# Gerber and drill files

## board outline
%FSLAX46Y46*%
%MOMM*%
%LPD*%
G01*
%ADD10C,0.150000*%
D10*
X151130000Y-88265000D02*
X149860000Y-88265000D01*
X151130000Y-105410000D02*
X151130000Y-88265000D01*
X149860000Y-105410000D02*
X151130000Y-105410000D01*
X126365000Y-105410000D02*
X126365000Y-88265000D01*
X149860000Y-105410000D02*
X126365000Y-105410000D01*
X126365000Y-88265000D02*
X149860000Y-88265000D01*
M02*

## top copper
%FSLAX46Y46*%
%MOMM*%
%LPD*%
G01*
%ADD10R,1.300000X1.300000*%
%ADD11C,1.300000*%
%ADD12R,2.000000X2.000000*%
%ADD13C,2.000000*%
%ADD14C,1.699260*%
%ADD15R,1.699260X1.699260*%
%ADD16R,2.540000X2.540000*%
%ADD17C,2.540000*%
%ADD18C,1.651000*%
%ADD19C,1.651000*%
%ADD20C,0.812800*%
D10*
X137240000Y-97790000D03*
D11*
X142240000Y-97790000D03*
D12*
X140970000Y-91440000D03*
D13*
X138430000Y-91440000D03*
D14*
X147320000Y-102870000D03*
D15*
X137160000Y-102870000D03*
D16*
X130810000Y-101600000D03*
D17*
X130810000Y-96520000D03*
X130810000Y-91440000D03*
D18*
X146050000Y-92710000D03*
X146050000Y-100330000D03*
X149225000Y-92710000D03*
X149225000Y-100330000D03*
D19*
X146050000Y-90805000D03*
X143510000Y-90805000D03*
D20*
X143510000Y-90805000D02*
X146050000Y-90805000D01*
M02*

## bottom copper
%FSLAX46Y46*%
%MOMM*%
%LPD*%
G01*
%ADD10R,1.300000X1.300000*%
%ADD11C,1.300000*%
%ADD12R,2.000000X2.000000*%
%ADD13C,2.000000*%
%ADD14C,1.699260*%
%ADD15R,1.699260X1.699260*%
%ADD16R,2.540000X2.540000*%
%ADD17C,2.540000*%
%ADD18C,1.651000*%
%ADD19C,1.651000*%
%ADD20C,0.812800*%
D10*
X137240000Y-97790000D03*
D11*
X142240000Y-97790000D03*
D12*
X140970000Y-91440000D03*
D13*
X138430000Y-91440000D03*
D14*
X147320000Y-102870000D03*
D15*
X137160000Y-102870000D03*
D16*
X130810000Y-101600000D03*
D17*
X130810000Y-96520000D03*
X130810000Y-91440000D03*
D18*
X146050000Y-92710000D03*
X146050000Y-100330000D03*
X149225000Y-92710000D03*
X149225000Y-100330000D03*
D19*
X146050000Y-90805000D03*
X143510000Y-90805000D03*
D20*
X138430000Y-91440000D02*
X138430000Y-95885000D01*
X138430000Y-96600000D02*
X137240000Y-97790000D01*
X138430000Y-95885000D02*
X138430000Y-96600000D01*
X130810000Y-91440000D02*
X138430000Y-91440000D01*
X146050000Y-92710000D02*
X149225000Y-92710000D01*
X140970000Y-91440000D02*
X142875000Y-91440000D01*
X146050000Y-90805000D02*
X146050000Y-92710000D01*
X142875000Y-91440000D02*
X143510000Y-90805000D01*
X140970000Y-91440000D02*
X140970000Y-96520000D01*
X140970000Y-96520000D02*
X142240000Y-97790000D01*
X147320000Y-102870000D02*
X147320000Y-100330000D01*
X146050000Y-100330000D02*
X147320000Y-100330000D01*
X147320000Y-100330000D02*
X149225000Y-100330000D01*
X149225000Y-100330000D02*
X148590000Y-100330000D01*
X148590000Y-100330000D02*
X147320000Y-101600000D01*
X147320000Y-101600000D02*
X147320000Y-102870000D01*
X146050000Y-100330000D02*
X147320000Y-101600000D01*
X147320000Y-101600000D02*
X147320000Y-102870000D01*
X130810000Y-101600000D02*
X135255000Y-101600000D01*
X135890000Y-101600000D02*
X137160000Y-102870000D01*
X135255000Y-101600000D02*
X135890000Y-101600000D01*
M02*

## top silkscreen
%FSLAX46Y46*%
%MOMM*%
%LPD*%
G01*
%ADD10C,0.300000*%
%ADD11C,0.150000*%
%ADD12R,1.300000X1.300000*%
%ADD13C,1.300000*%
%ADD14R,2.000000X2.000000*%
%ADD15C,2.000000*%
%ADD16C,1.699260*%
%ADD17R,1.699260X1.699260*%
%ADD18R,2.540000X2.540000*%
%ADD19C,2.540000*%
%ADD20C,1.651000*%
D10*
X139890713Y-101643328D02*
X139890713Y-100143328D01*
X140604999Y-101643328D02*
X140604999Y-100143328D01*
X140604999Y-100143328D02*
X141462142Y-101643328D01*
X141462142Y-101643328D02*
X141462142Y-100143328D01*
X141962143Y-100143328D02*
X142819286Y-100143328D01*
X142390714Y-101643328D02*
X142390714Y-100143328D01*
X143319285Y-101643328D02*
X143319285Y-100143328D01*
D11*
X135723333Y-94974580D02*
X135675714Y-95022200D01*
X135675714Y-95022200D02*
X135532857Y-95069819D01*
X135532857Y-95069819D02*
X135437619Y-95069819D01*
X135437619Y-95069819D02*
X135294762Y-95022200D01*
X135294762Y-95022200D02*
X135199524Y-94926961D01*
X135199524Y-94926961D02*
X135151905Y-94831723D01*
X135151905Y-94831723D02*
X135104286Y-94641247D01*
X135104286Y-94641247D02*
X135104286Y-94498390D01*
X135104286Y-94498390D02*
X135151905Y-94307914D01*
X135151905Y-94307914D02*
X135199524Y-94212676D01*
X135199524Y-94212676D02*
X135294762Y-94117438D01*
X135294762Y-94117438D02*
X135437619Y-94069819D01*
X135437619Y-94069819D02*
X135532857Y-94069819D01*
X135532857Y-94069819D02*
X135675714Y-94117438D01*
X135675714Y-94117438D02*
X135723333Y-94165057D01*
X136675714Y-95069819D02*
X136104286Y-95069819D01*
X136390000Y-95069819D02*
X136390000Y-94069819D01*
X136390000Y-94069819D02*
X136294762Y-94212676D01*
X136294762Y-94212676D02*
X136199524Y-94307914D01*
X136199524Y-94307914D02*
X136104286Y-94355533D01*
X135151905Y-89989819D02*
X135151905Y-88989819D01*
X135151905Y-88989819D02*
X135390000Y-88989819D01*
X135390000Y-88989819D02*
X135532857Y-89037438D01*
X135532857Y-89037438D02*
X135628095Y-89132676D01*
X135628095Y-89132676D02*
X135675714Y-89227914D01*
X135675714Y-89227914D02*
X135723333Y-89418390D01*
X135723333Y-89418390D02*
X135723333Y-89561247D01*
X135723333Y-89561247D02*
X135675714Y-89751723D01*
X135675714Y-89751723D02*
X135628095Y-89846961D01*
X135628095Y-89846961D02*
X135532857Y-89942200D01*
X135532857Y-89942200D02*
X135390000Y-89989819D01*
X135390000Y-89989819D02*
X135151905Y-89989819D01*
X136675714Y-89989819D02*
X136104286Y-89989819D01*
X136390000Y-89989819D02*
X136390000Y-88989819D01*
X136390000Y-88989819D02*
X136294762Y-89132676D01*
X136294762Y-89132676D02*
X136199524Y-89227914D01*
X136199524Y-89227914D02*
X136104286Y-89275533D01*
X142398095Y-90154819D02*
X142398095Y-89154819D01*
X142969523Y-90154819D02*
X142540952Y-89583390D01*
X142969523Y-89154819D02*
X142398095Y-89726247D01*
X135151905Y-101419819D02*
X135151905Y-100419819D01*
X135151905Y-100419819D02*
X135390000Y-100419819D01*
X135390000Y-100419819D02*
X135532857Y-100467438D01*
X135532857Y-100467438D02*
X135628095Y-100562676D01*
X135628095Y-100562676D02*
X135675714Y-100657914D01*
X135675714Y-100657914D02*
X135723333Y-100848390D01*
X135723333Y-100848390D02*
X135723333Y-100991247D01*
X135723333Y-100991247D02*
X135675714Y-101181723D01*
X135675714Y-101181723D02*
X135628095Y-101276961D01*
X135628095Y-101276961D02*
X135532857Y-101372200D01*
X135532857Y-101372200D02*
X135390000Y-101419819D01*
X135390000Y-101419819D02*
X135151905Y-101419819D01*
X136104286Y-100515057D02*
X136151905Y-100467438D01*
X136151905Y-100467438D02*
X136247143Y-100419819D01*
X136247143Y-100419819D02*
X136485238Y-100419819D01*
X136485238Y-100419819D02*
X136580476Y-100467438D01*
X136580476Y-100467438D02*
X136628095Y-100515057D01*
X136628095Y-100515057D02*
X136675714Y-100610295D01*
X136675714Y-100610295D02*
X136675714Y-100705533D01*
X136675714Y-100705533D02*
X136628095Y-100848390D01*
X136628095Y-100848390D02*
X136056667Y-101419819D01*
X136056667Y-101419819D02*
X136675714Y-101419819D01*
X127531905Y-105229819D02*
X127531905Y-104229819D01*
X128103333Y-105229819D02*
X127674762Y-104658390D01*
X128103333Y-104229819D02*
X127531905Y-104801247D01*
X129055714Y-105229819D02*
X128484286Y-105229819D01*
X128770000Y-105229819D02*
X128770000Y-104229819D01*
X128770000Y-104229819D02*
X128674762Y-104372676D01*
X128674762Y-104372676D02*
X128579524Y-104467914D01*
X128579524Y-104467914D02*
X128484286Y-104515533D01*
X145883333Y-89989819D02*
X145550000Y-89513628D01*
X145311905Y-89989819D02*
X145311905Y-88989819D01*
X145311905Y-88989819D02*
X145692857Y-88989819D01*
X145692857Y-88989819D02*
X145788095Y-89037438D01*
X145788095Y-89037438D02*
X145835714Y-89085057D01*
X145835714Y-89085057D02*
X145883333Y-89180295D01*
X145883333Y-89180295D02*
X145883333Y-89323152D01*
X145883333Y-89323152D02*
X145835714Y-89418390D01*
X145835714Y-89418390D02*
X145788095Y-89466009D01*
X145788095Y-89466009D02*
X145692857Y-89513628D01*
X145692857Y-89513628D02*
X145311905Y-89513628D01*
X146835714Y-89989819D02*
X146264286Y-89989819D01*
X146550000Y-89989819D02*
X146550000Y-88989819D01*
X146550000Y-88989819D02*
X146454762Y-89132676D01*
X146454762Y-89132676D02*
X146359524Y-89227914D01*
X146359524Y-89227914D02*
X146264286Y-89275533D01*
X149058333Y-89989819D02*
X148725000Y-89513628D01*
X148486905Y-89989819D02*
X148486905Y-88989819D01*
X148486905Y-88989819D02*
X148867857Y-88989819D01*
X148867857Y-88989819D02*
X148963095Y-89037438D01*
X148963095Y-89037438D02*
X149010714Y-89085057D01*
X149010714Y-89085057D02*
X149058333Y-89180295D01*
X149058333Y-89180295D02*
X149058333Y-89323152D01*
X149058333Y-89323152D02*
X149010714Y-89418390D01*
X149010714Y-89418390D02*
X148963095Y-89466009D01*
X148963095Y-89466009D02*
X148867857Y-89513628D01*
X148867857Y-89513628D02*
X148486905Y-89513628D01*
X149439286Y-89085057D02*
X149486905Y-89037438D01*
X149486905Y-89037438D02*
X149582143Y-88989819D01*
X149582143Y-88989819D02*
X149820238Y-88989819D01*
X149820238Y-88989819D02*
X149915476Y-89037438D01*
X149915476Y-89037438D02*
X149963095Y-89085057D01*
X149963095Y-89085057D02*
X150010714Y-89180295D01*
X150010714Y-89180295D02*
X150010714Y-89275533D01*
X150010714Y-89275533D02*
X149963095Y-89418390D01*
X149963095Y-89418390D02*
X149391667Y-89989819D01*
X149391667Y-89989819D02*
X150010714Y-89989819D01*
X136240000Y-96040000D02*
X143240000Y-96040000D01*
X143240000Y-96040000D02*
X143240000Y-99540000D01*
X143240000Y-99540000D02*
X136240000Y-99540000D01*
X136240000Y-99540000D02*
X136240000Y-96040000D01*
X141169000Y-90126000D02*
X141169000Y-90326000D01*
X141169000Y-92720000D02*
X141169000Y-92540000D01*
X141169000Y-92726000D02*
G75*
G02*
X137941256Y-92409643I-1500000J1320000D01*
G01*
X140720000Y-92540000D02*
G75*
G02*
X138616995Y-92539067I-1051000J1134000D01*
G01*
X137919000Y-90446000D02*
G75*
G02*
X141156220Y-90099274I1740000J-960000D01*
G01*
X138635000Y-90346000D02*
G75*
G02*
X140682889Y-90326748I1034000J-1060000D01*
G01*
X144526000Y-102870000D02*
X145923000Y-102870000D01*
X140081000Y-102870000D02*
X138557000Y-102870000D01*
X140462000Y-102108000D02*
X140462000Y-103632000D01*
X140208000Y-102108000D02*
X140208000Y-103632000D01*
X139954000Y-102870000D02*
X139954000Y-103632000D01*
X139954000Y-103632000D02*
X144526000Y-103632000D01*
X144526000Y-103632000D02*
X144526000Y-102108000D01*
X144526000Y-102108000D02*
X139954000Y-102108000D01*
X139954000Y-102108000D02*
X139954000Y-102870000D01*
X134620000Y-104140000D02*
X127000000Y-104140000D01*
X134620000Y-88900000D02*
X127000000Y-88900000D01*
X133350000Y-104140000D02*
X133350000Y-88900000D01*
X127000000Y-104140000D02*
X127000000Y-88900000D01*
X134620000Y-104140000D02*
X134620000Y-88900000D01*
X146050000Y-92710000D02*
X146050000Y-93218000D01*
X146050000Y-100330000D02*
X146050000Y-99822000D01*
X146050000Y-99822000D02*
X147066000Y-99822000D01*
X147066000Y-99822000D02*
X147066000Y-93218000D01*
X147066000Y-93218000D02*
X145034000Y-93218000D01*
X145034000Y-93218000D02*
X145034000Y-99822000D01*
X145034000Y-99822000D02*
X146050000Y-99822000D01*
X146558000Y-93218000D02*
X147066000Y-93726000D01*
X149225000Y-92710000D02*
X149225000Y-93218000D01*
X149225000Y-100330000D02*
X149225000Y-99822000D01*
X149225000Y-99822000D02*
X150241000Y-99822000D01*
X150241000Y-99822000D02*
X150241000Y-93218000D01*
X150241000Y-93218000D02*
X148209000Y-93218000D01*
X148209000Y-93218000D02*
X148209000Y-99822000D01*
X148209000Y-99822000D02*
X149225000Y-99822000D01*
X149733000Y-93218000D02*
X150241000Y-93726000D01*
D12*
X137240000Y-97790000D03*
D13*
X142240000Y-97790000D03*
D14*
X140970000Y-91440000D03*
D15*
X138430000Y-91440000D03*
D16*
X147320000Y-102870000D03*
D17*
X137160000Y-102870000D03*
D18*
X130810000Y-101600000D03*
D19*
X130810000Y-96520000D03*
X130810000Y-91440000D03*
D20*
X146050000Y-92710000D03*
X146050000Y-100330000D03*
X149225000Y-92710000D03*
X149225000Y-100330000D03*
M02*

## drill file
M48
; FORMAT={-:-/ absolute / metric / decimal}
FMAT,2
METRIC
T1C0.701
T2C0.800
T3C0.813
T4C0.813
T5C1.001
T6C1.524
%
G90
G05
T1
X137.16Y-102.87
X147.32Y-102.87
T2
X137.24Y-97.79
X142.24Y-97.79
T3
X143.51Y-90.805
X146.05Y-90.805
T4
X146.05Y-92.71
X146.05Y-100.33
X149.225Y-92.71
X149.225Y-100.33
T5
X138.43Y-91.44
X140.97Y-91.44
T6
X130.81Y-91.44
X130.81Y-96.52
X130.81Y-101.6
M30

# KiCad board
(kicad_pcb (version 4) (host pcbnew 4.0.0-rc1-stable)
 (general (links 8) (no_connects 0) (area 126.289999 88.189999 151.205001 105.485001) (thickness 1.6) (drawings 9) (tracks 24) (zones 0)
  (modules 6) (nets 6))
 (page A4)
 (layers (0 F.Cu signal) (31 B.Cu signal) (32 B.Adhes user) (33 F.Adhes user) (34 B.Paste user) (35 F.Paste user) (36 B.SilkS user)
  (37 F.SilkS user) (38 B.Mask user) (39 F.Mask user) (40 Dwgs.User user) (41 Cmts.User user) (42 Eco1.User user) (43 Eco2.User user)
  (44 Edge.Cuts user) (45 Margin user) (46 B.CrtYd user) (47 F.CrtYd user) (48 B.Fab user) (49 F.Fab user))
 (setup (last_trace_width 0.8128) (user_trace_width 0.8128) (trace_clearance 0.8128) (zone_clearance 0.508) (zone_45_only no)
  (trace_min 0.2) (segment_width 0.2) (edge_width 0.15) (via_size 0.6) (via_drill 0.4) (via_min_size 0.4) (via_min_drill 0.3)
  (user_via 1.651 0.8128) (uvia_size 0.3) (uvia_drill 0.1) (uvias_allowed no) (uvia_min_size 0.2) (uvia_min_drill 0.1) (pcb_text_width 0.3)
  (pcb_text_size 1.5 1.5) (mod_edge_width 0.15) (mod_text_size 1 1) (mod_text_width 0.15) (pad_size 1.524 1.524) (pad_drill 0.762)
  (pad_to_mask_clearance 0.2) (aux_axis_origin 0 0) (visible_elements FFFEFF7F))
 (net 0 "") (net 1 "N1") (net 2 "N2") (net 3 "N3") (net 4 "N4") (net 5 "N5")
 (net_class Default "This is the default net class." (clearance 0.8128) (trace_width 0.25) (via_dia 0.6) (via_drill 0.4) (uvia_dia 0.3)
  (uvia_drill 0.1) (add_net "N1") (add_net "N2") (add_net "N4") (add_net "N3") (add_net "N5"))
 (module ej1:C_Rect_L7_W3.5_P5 (layer F.Cu) (at 137.24 97.79)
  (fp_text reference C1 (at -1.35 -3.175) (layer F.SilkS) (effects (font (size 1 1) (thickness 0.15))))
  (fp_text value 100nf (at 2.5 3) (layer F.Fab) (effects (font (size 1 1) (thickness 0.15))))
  (fp_line (start -1 -1.75) (end 6 -1.75) (layer F.SilkS) (width 0.15))
  (fp_line (start 6 -1.75) (end 6 1.75) (layer F.SilkS) (width 0.15))
  (fp_line (start 6 1.75) (end -1 1.75) (layer F.SilkS) (width 0.15))
  (fp_line (start -1 1.75) (end -1 -1.75) (layer F.SilkS) (width 0.15))
  (pad 1 thru_hole rect (at 0 0) (size 1.3 1.3) (drill 0.8) (layers *.Cu *.Mask F.SilkS) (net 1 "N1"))
  (pad 2 thru_hole circle (at 5 0) (size 1.3 1.3) (drill 0.8) (layers *.Cu *.Mask F.SilkS) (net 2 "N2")))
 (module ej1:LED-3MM (layer F.Cu) (at 140.97 91.44 180)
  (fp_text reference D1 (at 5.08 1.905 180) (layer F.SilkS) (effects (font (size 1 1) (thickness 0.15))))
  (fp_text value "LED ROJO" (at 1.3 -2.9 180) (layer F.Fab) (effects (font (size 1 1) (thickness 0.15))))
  (fp_line (start -0.199 1.314) (end -0.199 1.114) (layer F.SilkS) (width 0.15))
  (fp_line (start -0.199 -1.28) (end -0.199 -1.1) (layer F.SilkS) (width 0.15))
  (fp_arc (start 1.301 0.034) (end -0.199 -1.286) (angle 108.5) (layer F.SilkS) (width 0.15))
  (fp_arc (start 1.301 0.034) (end 0.25 -1.1) (angle 85.7) (layer F.SilkS) (width 0.15))
  (fp_arc (start 1.311 0.034) (end 3.051 0.994) (angle 110) (layer F.SilkS) (width 0.15))
  (fp_arc (start 1.301 0.034) (end 2.335 1.094) (angle 87.5) (layer F.SilkS) (width 0.15))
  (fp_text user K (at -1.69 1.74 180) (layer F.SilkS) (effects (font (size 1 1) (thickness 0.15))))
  (pad 1 thru_hole rect (at 0 0 270) (size 2 2) (drill 1.00076) (layers *.Cu *.Mask F.SilkS) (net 2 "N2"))
  (pad 2 thru_hole circle (at 2.54 0 180) (size 2 2) (drill 1.00076) (layers *.Cu *.Mask F.SilkS) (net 1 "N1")))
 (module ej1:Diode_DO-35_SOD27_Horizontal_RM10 (layer F.Cu) (at 137.15948 102.87254)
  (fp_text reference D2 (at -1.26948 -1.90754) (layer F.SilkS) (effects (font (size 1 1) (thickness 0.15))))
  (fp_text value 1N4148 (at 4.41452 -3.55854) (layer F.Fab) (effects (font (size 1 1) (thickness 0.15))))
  (fp_line (start 7.36652 -0.00254) (end 8.76352 -0.00254) (layer F.SilkS) (width 0.15))
  (fp_line (start 2.92152 -0.00254) (end 1.39752 -0.00254) (layer F.SilkS) (width 0.15))
  (fp_line (start 3.30252 -0.76454) (end 3.30252 0.75946) (layer F.SilkS) (width 0.15))
  (fp_line (start 3.04852 -0.76454) (end 3.04852 0.75946) (layer F.SilkS) (width 0.15))
  (fp_line (start 2.79452 -0.00254) (end 2.79452 0.75946) (layer F.SilkS) (width 0.15))
  (fp_line (start 2.79452 0.75946) (end 7.36652 0.75946) (layer F.SilkS) (width 0.15))
  (fp_line (start 7.36652 0.75946) (end 7.36652 -0.76454) (layer F.SilkS) (width 0.15))
  (fp_line (start 7.36652 -0.76454) (end 2.79452 -0.76454) (layer F.SilkS) (width 0.15))
  (fp_line (start 2.79452 -0.76454) (end 2.79452 -0.00254) (layer F.SilkS) (width 0.15))
  (pad 2 thru_hole circle (at 10.16052 -0.00254 180) (size 1.69926 1.69926) (drill 0.70104) (layers *.Cu *.Mask F.SilkS) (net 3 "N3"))
  (pad 1 thru_hole rect (at 0.00052 -0.00254 180) (size 1.69926 1.69926) (drill 0.70104) (layers *.Cu *.Mask F.SilkS) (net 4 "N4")))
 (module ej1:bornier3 (layer F.Cu) (at 130.81 96.52 90)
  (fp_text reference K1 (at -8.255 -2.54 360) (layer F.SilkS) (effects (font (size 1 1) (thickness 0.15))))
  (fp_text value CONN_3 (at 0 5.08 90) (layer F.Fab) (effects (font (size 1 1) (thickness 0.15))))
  (fp_line (start -7.62 3.81) (end -7.62 -3.81) (layer F.SilkS) (width 0.15))
  (fp_line (start 7.62 3.81) (end 7.62 -3.81) (layer F.SilkS) (width 0.15))
  (fp_line (start -7.62 2.54) (end 7.62 2.54) (layer F.SilkS) (width 0.15))
  (fp_line (start -7.62 -3.81) (end 7.62 -3.81) (layer F.SilkS) (width 0.15))
  (fp_line (start -7.62 3.81) (end 7.62 3.81) (layer F.SilkS) (width 0.15))
  (pad 1 thru_hole rect (at -5.08 0 90) (size 2.54 2.54) (drill 1.524) (layers *.Cu *.Mask F.SilkS) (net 4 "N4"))
  (pad 2 thru_hole circle (at 0 0 90) (size 2.54 2.54) (drill 1.524) (layers *.Cu *.Mask F.SilkS) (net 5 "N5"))
  (pad 3 thru_hole circle (at 5.08 0 90) (size 2.54 2.54) (drill 1.524) (layers *.Cu *.Mask F.SilkS) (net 1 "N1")))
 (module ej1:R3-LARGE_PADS (layer F.Cu) (at 146.05 96.52 270)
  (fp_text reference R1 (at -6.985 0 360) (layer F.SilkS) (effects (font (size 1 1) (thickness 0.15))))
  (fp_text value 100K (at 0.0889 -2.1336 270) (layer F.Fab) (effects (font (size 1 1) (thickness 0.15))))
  (fp_line (start -3.81 0) (end -3.302 0) (layer F.SilkS) (width 0.15))
  (fp_line (start 3.81 0) (end 3.302 0) (layer F.SilkS) (width 0.15))
  (fp_line (start 3.302 0) (end 3.302 -1.016) (layer F.SilkS) (width 0.15))
  (fp_line (start 3.302 -1.016) (end -3.302 -1.016) (layer F.SilkS) (width 0.15))
  (fp_line (start -3.302 -1.016) (end -3.302 1.016) (layer F.SilkS) (width 0.15))
  (fp_line (start -3.302 1.016) (end 3.302 1.016) (layer F.SilkS) (width 0.15))
  (fp_line (start 3.302 1.016) (end 3.302 0) (layer F.SilkS) (width 0.15))
  (fp_line (start -3.302 -0.508) (end -2.794 -1.016) (layer F.SilkS) (width 0.15))
  (pad 1 thru_hole circle (at -3.81 0 270) (size 1.651 1.651) (drill 0.8128) (layers *.Cu *.Mask F.SilkS) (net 2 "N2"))
  (pad 2 thru_hole circle (at 3.81 0 270) (size 1.651 1.651) (drill 0.8128) (layers *.Cu *.Mask F.SilkS) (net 3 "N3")))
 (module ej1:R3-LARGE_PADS (layer F.Cu) (at 149.225 96.52 270)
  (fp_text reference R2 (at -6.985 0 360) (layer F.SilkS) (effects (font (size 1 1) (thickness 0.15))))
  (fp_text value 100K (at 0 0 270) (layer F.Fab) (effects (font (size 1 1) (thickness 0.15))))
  (fp_line (start -3.81 0) (end -3.302 0) (layer F.SilkS) (width 0.15))
  (fp_line (start 3.81 0) (end 3.302 0) (layer F.SilkS) (width 0.15))
  (fp_line (start 3.302 0) (end 3.302 -1.016) (layer F.SilkS) (width 0.15))
  (fp_line (start 3.302 -1.016) (end -3.302 -1.016) (layer F.SilkS) (width 0.15))
  (fp_line (start -3.302 -1.016) (end -3.302 1.016) (layer F.SilkS) (width 0.15))
  (fp_line (start -3.302 1.016) (end 3.302 1.016) (layer F.SilkS) (width 0.15))
  (fp_line (start 3.302 1.016) (end 3.302 0) (layer F.SilkS) (width 0.15))
  (fp_line (start -3.302 -0.508) (end -2.794 -1.016) (layer F.SilkS) (width 0.15))
  (pad 1 thru_hole circle (at -3.81 0 270) (size 1.651 1.651) (drill 0.8128) (layers *.Cu *.Mask F.SilkS) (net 2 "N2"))
  (pad 2 thru_hole circle (at 3.81 0 270) (size 1.651 1.651) (drill 0.8128) (layers *.Cu *.Mask F.SilkS) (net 3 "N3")))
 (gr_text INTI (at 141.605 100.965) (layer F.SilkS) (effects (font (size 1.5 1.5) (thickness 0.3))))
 (gr_line (start 151.13 88.265) (end 149.86 88.265) (angle 90) (layer Edge.Cuts) (width 0.15))
 (gr_line (start 151.13 105.41) (end 151.13 88.265) (angle 90) (layer Edge.Cuts) (width 0.15))
 (gr_line (start 149.86 105.41) (end 151.13 105.41) (angle 90) (layer Edge.Cuts) (width 0.15))
 (gr_line (start 126.365 105.41) (end 126.365 88.265) (angle 90) (layer Edge.Cuts) (width 0.15))
 (gr_line (start 149.86 105.41) (end 126.365 105.41) (angle 90) (layer Edge.Cuts) (width 0.15))
 (gr_line (start 126.365 88.265) (end 149.86 88.265) (angle 90) (layer Edge.Cuts) (width 0.15))
 (segment (start 138.43 91.44) (end 138.43 95.885) (width 0.8128) (layer B.Cu) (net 1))
 (segment (start 138.43 96.6) (end 137.24 97.79) (width 0.8128) (layer B.Cu) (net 1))
 (segment (start 138.43 95.885) (end 138.43 96.6) (width 0.8128) (layer B.Cu) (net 1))
 (segment (start 130.81 91.44) (end 138.43 91.44) (width 0.8128) (layer B.Cu) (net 1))
 (segment (start 146.05 92.71) (end 149.225 92.71) (width 0.8128) (layer B.Cu) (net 2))
 (segment (start 140.97 91.44) (end 142.875 91.44) (width 0.8128) (layer B.Cu) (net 2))
 (segment (start 146.05 90.805) (end 146.05 92.71) (width 0.8128) (layer B.Cu) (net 2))
 (via (at 146.05 90.805) (size 1.651) (drill 0.8128) (layers F.Cu B.Cu) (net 2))
 (segment (start 143.51 90.805) (end 146.05 90.805) (width 0.8128) (layer F.Cu) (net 2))
 (via (at 143.51 90.805) (size 1.651) (drill 0.8128) (layers F.Cu B.Cu) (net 2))
 (segment (start 142.875 91.44) (end 143.51 90.805) (width 0.8128) (layer B.Cu) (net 2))
 (segment (start 140.97 91.44) (end 140.97 96.52) (width 0.8128) (layer B.Cu) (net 2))
 (segment (start 140.97 96.52) (end 142.24 97.79) (width 0.8128) (layer B.Cu) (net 2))
 (segment (start 147.32 102.87) (end 147.32 100.33) (width 0.8128) (layer B.Cu) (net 3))
 (segment (start 146.05 100.33) (end 147.32 100.33) (width 0.8128) (layer B.Cu) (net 3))
 (segment (start 147.32 100.33) (end 149.225 100.33) (width 0.8128) (layer B.Cu) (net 3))
 (segment (start 149.225 100.33) (end 148.59 100.33) (width 0.8128) (layer B.Cu) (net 3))
 (segment (start 148.59 100.33) (end 147.32 101.6) (width 0.8128) (layer B.Cu) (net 3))
 (segment (start 147.32 101.6) (end 147.32 102.87) (width 0.8128) (layer B.Cu) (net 3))
 (segment (start 146.05 100.33) (end 147.32 101.6) (width 0.8128) (layer B.Cu) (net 3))
 (segment (start 147.32 101.6) (end 147.32 102.87) (width 0.8128) (layer B.Cu) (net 3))
 (segment (start 130.81 101.6) (end 135.255 101.6) (width 0.8128) (layer B.Cu) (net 4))
 (segment (start 135.89 101.6) (end 137.16 102.87) (width 0.8128) (layer B.Cu) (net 4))
 (segment (start 135.255 101.6) (end 135.89 101.6) (width 0.8128) (layer B.Cu) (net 4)))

